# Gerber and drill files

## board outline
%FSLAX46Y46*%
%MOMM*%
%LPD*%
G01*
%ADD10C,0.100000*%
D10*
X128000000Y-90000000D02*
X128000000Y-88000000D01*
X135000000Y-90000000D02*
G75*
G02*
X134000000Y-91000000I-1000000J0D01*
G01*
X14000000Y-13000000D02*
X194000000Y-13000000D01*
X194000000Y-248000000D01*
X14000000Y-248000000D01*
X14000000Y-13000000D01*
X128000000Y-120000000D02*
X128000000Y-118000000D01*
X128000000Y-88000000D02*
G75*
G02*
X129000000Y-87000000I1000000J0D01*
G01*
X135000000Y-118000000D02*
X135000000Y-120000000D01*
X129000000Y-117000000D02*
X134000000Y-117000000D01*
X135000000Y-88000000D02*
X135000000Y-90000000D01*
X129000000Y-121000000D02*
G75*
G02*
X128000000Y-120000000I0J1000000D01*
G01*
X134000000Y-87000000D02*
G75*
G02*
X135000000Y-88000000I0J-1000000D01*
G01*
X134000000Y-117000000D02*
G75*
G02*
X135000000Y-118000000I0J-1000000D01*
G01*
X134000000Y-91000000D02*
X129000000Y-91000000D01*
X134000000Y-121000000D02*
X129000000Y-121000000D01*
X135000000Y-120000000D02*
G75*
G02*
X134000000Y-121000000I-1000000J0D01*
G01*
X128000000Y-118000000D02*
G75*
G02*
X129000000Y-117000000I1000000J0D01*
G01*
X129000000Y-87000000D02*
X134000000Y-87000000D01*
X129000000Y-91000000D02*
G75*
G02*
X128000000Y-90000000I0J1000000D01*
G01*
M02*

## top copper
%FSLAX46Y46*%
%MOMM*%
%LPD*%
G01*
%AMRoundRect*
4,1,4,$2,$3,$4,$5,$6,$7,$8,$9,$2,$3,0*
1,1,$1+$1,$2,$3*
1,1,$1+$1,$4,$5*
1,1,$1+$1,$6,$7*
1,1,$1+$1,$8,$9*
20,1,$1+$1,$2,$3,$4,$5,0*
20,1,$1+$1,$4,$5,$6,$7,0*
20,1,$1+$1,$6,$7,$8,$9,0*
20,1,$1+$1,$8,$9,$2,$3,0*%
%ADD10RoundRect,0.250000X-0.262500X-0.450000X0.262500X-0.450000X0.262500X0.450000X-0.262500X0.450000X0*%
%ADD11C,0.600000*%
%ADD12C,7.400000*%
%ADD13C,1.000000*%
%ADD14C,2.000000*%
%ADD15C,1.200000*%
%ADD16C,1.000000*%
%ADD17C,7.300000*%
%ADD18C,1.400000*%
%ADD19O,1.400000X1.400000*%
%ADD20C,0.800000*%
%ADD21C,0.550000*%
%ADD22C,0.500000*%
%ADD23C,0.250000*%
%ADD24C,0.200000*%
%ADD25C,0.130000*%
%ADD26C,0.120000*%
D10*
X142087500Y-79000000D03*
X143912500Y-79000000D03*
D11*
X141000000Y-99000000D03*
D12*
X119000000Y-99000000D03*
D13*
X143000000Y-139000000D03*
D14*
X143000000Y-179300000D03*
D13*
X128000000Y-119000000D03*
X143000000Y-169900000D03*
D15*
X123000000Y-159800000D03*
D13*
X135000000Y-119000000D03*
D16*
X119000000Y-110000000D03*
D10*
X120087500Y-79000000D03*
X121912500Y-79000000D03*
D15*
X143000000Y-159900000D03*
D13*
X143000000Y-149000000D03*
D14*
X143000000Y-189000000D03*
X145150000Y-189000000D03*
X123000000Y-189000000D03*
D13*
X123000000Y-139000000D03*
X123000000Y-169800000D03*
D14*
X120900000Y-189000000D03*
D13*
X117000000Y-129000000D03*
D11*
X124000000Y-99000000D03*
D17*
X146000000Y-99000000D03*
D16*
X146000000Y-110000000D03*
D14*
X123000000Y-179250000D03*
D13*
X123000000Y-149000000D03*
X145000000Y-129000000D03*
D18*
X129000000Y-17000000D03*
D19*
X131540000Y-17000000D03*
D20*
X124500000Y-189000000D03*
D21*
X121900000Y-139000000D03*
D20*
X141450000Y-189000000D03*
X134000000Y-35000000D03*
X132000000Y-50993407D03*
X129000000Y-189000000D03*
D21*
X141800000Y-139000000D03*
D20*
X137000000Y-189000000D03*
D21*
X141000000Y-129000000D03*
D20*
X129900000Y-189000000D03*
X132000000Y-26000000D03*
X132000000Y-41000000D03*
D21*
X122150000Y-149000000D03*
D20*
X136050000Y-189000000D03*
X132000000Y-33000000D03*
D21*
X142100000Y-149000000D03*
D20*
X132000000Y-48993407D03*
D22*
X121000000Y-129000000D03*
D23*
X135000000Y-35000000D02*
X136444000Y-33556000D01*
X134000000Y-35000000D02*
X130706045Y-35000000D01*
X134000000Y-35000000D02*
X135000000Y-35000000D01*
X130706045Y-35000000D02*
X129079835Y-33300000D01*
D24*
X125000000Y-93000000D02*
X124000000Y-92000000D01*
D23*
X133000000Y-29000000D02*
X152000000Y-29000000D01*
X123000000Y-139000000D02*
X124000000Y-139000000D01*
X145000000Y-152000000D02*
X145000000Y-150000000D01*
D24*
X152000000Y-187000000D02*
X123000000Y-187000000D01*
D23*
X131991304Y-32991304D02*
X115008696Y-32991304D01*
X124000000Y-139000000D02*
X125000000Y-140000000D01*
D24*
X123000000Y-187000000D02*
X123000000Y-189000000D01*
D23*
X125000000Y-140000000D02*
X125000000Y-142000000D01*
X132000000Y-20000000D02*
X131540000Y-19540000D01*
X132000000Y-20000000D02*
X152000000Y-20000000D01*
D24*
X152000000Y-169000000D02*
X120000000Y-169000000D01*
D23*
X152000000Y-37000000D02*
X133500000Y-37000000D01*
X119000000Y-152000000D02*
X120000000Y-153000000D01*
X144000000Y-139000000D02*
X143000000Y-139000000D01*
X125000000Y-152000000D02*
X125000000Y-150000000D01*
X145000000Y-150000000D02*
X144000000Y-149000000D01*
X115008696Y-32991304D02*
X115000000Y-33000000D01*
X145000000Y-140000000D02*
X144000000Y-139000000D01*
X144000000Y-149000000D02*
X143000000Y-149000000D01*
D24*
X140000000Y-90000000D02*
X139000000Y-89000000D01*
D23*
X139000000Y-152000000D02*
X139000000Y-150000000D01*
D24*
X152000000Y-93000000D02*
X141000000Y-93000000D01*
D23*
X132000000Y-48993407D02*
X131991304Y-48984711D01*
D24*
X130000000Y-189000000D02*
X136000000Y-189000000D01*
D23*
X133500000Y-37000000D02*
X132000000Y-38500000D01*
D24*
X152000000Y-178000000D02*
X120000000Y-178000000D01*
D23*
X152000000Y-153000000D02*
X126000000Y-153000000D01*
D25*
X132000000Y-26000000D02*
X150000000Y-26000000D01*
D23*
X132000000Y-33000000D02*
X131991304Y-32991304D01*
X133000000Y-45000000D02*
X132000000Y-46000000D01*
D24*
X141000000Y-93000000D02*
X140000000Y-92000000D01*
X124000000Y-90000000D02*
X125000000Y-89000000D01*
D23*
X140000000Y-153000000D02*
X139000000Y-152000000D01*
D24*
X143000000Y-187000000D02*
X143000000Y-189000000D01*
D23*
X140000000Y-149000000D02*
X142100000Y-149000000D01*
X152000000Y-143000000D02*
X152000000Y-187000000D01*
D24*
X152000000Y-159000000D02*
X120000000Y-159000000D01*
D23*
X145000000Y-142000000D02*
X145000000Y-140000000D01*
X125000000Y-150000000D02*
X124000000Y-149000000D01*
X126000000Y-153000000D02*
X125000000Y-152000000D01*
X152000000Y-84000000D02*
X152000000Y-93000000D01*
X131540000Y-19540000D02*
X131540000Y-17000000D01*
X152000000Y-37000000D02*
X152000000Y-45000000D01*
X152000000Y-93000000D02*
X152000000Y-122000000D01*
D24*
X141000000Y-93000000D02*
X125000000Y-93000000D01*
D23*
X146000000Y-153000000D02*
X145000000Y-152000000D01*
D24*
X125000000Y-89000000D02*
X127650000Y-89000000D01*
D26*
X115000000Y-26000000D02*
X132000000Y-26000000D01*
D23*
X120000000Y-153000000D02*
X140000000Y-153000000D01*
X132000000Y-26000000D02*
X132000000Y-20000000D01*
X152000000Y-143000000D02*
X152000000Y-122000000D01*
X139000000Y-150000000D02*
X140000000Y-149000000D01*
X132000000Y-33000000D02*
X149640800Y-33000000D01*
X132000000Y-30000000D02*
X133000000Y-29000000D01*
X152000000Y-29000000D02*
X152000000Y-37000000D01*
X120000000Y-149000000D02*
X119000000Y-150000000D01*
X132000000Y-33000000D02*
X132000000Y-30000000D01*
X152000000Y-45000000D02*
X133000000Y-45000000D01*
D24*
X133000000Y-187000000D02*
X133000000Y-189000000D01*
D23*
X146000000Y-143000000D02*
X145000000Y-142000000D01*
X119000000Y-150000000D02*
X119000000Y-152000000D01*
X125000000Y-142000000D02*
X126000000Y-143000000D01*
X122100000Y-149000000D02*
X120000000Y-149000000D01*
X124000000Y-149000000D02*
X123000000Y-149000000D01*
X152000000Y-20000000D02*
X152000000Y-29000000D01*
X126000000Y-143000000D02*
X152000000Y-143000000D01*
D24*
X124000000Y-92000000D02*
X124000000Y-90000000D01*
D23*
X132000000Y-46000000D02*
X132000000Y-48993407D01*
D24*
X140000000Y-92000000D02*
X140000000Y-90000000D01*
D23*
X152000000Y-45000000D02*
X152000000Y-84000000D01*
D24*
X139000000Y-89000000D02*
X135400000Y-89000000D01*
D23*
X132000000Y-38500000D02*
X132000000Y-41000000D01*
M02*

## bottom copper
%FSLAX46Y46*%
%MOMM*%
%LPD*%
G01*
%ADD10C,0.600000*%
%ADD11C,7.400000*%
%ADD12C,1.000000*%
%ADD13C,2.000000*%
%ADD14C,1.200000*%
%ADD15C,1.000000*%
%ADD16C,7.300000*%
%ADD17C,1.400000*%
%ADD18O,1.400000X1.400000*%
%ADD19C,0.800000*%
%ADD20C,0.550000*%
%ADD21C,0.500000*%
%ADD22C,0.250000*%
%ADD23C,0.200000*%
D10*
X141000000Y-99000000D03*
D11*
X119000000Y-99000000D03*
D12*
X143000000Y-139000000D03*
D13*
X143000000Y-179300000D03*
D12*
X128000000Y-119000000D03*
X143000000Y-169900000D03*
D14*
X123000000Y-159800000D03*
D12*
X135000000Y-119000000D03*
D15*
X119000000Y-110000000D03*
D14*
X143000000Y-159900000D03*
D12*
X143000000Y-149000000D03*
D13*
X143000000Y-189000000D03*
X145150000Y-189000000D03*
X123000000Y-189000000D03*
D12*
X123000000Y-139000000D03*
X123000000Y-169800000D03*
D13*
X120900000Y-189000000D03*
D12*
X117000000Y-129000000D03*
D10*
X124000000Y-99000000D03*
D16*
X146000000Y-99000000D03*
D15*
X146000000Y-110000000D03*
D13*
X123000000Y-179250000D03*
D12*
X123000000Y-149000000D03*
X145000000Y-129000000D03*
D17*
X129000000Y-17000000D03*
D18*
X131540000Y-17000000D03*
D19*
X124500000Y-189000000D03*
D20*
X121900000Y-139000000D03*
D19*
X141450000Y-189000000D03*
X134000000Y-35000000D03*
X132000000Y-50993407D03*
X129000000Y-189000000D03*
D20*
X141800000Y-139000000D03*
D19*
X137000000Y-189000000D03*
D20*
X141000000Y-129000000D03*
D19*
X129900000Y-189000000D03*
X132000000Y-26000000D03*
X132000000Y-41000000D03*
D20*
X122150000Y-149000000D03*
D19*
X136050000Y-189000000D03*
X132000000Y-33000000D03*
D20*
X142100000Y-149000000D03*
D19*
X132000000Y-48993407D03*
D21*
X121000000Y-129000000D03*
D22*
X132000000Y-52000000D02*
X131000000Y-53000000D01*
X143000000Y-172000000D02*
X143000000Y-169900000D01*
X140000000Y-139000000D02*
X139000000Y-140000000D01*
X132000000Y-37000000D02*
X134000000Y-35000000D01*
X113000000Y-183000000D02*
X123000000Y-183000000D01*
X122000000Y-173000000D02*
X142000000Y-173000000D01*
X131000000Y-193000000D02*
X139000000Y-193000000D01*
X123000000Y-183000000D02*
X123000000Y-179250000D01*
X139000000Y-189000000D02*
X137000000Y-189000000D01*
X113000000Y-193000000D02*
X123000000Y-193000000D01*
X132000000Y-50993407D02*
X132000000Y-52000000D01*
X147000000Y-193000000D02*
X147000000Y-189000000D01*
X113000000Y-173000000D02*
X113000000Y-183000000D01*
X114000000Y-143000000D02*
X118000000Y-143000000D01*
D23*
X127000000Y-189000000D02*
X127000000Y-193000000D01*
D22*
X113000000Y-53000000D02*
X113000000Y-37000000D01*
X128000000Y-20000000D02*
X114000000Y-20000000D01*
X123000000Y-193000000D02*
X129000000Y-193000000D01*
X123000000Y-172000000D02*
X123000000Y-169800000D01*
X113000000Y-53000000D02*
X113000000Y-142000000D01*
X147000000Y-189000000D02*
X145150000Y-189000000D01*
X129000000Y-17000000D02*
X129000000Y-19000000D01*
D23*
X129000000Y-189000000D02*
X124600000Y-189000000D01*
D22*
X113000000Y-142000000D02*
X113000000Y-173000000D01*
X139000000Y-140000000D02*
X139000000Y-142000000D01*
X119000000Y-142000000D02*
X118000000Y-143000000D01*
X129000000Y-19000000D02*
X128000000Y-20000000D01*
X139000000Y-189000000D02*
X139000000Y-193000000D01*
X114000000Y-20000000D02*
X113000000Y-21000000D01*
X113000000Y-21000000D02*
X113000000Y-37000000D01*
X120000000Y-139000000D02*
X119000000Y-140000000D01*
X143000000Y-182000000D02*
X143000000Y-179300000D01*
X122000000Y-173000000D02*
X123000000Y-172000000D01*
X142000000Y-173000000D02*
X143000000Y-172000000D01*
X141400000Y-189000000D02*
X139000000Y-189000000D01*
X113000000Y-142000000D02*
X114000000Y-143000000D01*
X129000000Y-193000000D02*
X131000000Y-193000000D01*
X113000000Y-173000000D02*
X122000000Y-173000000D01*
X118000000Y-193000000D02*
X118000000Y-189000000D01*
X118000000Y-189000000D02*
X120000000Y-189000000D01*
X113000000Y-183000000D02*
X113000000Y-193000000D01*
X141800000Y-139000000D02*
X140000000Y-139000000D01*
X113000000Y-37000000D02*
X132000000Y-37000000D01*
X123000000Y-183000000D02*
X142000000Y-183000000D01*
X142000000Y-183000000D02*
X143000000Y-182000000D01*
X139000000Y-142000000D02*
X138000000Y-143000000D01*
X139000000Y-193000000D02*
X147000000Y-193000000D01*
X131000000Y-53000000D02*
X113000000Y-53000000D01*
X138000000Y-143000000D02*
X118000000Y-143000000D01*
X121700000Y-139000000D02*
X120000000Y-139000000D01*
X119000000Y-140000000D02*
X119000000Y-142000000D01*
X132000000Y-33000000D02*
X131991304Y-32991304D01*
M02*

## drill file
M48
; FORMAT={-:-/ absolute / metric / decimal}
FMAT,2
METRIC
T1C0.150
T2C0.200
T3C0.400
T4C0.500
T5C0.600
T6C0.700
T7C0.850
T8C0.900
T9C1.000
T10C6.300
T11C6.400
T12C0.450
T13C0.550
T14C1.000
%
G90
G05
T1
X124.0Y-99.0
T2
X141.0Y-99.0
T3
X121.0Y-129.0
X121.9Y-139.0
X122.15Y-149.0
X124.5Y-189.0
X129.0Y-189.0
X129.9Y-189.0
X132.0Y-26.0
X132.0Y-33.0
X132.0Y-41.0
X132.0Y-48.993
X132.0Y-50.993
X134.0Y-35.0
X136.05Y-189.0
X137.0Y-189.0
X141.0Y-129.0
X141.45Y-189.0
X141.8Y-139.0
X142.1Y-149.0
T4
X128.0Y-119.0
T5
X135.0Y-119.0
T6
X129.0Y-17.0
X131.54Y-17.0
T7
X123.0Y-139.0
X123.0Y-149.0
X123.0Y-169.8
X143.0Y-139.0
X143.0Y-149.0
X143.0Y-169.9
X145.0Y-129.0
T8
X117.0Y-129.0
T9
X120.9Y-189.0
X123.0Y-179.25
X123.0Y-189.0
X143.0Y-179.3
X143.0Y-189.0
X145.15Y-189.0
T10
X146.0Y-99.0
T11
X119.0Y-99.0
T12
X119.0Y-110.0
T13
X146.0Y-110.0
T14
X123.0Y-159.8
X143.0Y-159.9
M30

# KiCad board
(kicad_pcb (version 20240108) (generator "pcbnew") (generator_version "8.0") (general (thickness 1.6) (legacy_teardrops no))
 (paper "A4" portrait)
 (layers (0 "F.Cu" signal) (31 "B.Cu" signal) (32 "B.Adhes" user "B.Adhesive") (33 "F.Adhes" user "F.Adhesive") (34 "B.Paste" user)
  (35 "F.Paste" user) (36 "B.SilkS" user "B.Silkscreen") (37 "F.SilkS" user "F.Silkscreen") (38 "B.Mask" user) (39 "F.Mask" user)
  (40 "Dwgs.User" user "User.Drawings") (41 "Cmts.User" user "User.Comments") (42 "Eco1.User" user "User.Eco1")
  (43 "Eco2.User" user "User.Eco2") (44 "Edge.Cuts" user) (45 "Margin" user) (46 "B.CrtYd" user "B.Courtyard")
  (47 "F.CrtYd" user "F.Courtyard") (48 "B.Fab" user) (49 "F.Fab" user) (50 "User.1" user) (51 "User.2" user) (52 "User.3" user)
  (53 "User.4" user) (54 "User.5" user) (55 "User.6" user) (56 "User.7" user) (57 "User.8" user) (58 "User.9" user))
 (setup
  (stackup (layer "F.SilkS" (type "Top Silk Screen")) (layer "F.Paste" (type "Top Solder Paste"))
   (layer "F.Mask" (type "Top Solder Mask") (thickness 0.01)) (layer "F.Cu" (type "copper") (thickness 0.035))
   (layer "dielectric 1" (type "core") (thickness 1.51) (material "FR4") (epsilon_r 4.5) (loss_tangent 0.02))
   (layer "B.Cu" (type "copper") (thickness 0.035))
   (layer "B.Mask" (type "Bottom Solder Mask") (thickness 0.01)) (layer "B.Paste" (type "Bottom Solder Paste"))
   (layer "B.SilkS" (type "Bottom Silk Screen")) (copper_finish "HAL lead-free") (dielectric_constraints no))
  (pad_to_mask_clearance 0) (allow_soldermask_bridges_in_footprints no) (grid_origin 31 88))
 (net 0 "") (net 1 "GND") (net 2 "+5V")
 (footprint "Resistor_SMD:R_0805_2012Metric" (layer "F.Cu") (at 143 79)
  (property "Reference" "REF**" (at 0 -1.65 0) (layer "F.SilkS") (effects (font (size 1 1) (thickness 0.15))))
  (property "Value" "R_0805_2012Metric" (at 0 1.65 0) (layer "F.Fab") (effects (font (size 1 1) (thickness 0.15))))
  (pad "1" smd roundrect (at -0.9125 0) (size 1.025 1.4) (layers "F.Cu" "F.Paste" "F.Mask") (roundrect_rratio 0.243902))
  (pad "2" smd roundrect (at 0.9125 0) (size 1.025 1.4) (layers "F.Cu" "F.Paste" "F.Mask") (roundrect_rratio 0.243902)))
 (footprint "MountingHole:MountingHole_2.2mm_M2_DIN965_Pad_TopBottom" (layer "F.Cu") (at 141 99)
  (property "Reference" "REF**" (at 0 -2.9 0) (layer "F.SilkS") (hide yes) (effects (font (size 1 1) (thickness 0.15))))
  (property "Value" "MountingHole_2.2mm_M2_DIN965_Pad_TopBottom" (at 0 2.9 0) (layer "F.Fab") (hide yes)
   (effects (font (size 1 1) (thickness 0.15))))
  (pad "1" thru_hole circle (at 0 0) (size 0.6 0.6) (drill 0.2) (layers "*.Cu" "*.Mask") (remove_unused_layers no)))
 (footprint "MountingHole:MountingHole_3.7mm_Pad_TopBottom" (layer "F.Cu") (at 119 99)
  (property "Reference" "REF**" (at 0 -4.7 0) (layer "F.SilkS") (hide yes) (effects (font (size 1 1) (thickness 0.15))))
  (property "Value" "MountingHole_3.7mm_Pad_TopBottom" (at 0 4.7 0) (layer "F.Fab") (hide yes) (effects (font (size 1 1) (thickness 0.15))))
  (pad "1" thru_hole circle (at 0 0) (size 7.4 7.4) (drill 6.4) (layers "*.Cu" "*.Mask") (remove_unused_layers no)))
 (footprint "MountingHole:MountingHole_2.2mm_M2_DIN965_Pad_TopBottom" (layer "F.Cu") (at 143 139)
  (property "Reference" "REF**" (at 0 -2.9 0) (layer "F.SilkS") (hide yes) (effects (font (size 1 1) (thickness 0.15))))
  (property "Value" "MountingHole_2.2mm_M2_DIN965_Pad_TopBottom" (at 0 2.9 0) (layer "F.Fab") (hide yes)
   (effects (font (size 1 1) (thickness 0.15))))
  (pad "1" thru_hole circle (at 0 0) (size 1 1) (drill 0.85) (layers "*.Cu" "*.Mask") (remove_unused_layers no) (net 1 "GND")))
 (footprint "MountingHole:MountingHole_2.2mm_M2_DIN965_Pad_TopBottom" (layer "F.Cu") (at 143 179.3)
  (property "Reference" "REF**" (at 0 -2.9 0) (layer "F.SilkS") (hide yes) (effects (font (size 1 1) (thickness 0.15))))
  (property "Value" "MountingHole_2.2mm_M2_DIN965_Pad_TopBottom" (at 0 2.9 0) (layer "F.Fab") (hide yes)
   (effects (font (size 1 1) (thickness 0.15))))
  (pad "1" thru_hole circle (at 0 0) (size 2 2) (drill 1) (layers "*.Cu" "*.Mask") (remove_unused_layers no) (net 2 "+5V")))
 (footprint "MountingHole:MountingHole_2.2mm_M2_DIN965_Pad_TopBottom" (layer "F.Cu") (at 128 119)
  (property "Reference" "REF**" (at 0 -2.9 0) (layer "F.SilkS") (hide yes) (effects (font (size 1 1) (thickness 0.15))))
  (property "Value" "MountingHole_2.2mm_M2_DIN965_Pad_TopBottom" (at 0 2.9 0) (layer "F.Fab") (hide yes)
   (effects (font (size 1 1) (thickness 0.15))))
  (pad "1" thru_hole circle (at 0 0) (size 1 1) (drill 0.5) (layers "*.Cu" "*.Mask") (remove_unused_layers no)))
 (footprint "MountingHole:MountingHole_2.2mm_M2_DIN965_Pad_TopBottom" (layer "F.Cu") (at 143 169.9)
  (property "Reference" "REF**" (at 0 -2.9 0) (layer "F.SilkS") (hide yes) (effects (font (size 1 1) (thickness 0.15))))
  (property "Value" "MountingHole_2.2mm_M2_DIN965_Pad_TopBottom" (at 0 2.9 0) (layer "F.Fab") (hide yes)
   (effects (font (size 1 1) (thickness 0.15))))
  (pad "1" thru_hole circle (at 0 0) (size 1 1) (drill 0.85) (layers "*.Cu" "*.Mask") (remove_unused_layers no) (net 2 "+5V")))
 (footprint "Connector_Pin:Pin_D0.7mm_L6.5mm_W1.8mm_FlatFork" (layer "F.Cu") (at 123 159.8)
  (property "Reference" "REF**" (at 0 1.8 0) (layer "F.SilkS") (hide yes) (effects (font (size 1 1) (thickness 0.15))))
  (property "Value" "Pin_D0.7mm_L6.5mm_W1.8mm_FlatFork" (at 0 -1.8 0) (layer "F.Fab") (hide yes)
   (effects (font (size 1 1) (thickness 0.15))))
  (pad "" np_thru_hole circle (at 0 0) (size 1.2 1.2) (drill 1) (layers "*.Cu" "*.Mask")))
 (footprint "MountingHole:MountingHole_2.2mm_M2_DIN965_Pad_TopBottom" (layer "F.Cu") (at 135 119)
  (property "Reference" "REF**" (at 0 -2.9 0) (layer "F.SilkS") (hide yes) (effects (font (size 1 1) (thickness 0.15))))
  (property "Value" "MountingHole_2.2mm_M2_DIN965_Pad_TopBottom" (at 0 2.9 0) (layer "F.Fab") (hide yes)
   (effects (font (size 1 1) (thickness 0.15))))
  (pad "1" thru_hole circle (at 0 0) (size 1 1) (drill 0.6) (layers "*.Cu" "*.Mask") (remove_unused_layers no)))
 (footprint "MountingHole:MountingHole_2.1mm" (layer "F.Cu") (at 119 110)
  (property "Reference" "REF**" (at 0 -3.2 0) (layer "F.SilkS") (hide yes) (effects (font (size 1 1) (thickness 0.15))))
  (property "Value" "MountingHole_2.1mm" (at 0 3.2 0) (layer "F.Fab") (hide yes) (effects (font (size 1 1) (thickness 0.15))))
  (pad "" np_thru_hole circle (at 0 0) (size 1 1) (drill 0.45) (layers "*.Cu" "*.Mask")))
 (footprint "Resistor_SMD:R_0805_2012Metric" (layer "F.Cu") (at 121 79)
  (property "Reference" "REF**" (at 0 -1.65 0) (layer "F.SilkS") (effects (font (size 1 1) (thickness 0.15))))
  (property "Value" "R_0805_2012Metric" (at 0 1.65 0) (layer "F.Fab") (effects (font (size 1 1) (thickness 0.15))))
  (pad "1" smd roundrect (at -0.9125 0) (size 1.025 1.4) (layers "F.Cu" "F.Paste" "F.Mask") (roundrect_rratio 0.243902))
  (pad "2" smd roundrect (at 0.9125 0) (size 1.025 1.4) (layers "F.Cu" "F.Paste" "F.Mask") (roundrect_rratio 0.243902)))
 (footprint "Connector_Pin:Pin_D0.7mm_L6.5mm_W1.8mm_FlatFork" (layer "F.Cu") (at 143 159.9)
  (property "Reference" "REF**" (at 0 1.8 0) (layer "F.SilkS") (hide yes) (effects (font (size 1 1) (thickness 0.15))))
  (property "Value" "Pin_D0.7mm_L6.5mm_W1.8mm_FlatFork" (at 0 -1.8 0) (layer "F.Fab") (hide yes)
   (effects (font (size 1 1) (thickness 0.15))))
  (pad "" np_thru_hole circle (at 0 0) (size 1.2 1.2) (drill 1) (layers "*.Cu" "*.Mask")))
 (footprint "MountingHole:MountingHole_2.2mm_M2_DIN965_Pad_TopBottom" (layer "F.Cu") (at 143 149)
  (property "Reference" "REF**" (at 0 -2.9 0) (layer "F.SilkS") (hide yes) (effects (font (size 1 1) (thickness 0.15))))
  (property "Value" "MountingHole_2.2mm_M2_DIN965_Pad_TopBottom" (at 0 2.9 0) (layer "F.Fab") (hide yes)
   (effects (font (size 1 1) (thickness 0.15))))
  (pad "1" thru_hole circle (at 0 0) (size 1 1) (drill 0.85) (layers "*.Cu" "*.Mask") (remove_unused_layers no) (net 1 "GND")))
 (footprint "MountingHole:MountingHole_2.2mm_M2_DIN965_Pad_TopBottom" (layer "F.Cu") (at 143 189)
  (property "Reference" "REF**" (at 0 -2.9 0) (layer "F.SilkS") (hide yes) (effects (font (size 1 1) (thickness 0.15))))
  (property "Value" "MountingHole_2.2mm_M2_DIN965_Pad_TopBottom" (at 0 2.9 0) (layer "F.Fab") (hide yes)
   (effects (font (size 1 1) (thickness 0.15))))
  (pad "1" thru_hole circle (at 0 0) (size 2 2) (drill 1) (layers "*.Cu" "*.Mask") (remove_unused_layers no) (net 1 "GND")))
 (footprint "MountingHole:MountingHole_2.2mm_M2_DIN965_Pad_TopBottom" (layer "F.Cu") (at 145.15 189)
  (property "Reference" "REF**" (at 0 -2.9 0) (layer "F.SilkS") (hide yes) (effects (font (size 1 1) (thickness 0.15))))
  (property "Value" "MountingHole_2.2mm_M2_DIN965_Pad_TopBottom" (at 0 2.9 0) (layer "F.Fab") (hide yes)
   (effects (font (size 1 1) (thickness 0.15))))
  (pad "1" thru_hole circle (at 0 0) (size 2 2) (drill 1) (layers "*.Cu" "*.Mask") (remove_unused_layers no) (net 2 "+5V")))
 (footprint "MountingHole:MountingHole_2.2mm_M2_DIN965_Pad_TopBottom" (layer "F.Cu") (at 123 189)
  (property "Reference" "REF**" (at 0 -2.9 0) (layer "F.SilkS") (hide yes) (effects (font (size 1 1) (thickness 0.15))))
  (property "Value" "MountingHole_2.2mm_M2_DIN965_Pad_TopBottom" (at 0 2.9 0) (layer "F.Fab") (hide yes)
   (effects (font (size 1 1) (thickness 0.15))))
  (pad "1" thru_hole circle (at 0 0) (size 2 2) (drill 1) (layers "*.Cu" "*.Mask") (remove_unused_layers no) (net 1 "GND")))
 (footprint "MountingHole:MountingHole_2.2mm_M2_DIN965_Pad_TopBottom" (layer "F.Cu") (at 123 139)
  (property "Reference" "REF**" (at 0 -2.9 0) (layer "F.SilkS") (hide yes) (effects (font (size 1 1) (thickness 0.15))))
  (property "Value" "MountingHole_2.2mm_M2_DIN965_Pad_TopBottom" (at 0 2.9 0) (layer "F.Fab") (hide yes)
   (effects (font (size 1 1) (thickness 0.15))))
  (pad "1" thru_hole circle (at 0 0) (size 1 1) (drill 0.85) (layers "*.Cu" "*.Mask") (remove_unused_layers no) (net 1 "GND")))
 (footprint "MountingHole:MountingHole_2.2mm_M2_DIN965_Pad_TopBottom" (layer "F.Cu") (at 123 169.8)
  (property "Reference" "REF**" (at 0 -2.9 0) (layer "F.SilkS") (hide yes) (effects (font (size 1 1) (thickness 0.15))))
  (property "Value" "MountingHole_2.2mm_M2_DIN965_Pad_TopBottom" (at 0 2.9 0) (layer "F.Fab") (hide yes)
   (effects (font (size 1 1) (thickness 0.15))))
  (pad "1" thru_hole circle (at 0 0) (size 1 1) (drill 0.85) (layers "*.Cu" "*.Mask") (remove_unused_layers no) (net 2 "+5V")))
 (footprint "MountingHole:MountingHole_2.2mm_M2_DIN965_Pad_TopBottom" (layer "F.Cu") (at 120.9 189)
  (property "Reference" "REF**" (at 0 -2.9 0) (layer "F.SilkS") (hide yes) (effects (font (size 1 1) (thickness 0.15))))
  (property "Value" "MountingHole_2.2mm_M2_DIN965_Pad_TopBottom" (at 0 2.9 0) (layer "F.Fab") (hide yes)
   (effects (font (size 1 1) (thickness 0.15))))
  (pad "1" thru_hole circle (at 0 0) (size 2 2) (drill 1) (layers "*.Cu" "*.Mask") (remove_unused_layers no) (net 2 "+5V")))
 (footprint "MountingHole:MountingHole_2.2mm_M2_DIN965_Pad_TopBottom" (layer "F.Cu") (at 117 129)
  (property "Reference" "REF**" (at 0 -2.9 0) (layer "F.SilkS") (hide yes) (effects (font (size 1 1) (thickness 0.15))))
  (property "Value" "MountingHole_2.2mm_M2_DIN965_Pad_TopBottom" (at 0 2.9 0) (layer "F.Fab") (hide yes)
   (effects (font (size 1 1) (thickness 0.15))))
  (pad "1" thru_hole circle (at 0 0) (size 1 1) (drill 0.9) (layers "*.Cu" "*.Mask") (remove_unused_layers no) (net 1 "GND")))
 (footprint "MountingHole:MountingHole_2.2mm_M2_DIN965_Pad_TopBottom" (layer "F.Cu") (at 124 99)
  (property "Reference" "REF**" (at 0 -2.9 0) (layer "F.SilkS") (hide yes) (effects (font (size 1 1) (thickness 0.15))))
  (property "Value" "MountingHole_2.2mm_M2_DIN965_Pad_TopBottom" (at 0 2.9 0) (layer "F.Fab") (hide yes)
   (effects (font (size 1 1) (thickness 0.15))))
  (pad "1" thru_hole circle (at 0 0) (size 0.6 0.6) (drill 0.15) (layers "*.Cu" "*.Mask") (remove_unused_layers no)))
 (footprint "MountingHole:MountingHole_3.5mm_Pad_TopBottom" (layer "F.Cu") (at 146 99)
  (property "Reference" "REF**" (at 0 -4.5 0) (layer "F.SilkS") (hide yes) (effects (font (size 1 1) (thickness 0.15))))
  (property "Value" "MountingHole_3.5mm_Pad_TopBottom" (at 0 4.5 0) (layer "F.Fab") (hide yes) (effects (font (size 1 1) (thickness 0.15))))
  (pad "1" thru_hole circle (at 0 0) (size 7.3 7.3) (drill 6.3) (layers "*.Cu" "*.Mask") (remove_unused_layers no)))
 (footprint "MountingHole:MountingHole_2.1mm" (layer "F.Cu") (at 146 110)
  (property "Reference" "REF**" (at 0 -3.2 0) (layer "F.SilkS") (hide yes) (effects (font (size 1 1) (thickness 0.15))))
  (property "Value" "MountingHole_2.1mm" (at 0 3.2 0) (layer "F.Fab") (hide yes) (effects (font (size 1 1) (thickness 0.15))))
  (pad "" np_thru_hole circle (at 0 0) (size 1 1) (drill 0.55) (layers "*.Cu" "*.Mask")))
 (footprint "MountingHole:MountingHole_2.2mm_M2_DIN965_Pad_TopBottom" (layer "F.Cu") (at 123 179.25)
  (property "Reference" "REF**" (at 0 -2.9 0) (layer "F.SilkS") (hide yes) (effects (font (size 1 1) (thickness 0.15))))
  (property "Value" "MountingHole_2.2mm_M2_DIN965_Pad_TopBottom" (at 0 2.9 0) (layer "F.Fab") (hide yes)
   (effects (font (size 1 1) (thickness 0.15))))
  (pad "1" thru_hole circle (at 0 0) (size 2 2) (drill 1) (layers "*.Cu" "*.Mask") (remove_unused_layers no) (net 2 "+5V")))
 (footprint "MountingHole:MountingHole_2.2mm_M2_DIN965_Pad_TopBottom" (layer "F.Cu") (at 123 149)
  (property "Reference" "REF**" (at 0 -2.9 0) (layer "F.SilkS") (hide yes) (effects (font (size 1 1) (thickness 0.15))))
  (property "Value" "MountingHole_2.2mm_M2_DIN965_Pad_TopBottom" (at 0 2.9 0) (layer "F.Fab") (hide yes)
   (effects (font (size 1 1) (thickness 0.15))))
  (pad "1" thru_hole circle (at 0 0) (size 1 1) (drill 0.85) (layers "*.Cu" "*.Mask") (remove_unused_layers no) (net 1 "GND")))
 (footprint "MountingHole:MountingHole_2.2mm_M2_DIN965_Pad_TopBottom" (layer "F.Cu") (at 145 129)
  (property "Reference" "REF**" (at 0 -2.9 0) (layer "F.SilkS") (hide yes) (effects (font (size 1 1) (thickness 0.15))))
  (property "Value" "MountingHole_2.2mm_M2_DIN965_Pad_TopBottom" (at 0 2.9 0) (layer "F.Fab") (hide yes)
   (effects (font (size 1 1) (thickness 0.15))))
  (pad "1" thru_hole circle (at 0 0) (size 1 1) (drill 0.85) (layers "*.Cu" "*.Mask") (remove_unused_layers no) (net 1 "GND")))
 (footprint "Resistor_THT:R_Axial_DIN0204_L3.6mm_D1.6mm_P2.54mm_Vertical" (layer "F.Cu") (at 129 17)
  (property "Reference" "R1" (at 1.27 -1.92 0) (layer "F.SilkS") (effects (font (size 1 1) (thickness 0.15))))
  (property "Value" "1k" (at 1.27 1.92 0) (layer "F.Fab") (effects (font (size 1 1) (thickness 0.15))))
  (pad "1" thru_hole circle (at 0 0) (size 1.4 1.4) (drill 0.7) (layers "*.Cu" "*.Mask") (remove_unused_layers no) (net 2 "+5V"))
  (pad "2" thru_hole oval (at 2.54 0) (size 1.4 1.4) (drill 0.7) (layers "*.Cu" "*.Mask") (remove_unused_layers no) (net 1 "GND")))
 (gr_line (start 128 90) (end 128 88) (stroke (width 0.1) (type default)) (layer "Edge.Cuts"))
 (gr_arc (start 135 90) (mid 134.707107 90.707107) (end 134 91) (stroke (width 0.1) (type default)) (layer "Edge.Cuts"))
 (gr_rect (start 14 13) (end 194 248) (locked yes) (stroke (width 0.1) (type default)) (fill none) (layer "Edge.Cuts"))
 (gr_line (start 128 120) (end 128 118) (stroke (width 0.1) (type default)) (layer "Edge.Cuts"))
 (gr_arc (start 128 88) (mid 128.292893 87.292893) (end 129 87) (stroke (width 0.1) (type default)) (layer "Edge.Cuts"))
 (gr_line (start 135 118) (end 135 120) (stroke (width 0.1) (type default)) (layer "Edge.Cuts"))
 (gr_line (start 129 117) (end 134 117) (stroke (width 0.1) (type default)) (layer "Edge.Cuts"))
 (gr_line (start 135 88) (end 135 90) (stroke (width 0.1) (type default)) (layer "Edge.Cuts"))
 (gr_arc (start 129 121) (mid 128.292893 120.707107) (end 128 120) (stroke (width 0.1) (type default)) (layer "Edge.Cuts"))
 (gr_arc (start 134 87) (mid 134.707107 87.292893) (end 135 88) (stroke (width 0.1) (type default)) (layer "Edge.Cuts"))
 (gr_arc (start 134 117) (mid 134.707107 117.292893) (end 135 118) (stroke (width 0.1) (type default)) (layer "Edge.Cuts"))
 (gr_line (start 134 91) (end 129 91) (stroke (width 0.1) (type default)) (layer "Edge.Cuts"))
 (gr_line (start 134 121) (end 129 121) (stroke (width 0.1) (type default)) (layer "Edge.Cuts"))
 (gr_arc (start 135 120) (mid 134.707107 120.707107) (end 134 121) (stroke (width 0.1) (type default)) (layer "Edge.Cuts"))
 (gr_arc (start 128 118) (mid 128.292893 117.292893) (end 129 117) (stroke (width 0.1) (type default)) (layer "Edge.Cuts"))
 (gr_line (start 129 87) (end 134 87) (stroke (width 0.1) (type default)) (layer "Edge.Cuts"))
 (gr_arc (start 129 91) (mid 128.292893 90.707107) (end 128 90) (stroke (width 0.1) (type default)) (layer "Edge.Cuts"))
 (segment (start 135 35) (end 136.444 33.556) (width 0.25) (layer "F.Cu") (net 2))
 (segment (start 134 35) (end 130.706045 35) (width 0.25) (layer "F.Cu") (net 2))
 (segment (start 134 35) (end 135 35) (width 0.25) (layer "F.Cu") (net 2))
 (segment (start 130.706045 35) (end 129.079835 33.3) (width 0.25) (layer "F.Cu") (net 2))
 (via (at 124.5 189) (size 0.8) (drill 0.4) (layers "F.Cu" "B.Cu") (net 2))
 (via (at 121.9 139) (size 0.55) (drill 0.4) (layers "F.Cu" "B.Cu") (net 2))
 (via (at 141.45 189) (size 0.8) (drill 0.4) (layers "F.Cu" "B.Cu") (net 2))
 (via (at 134 35) (size 0.8) (drill 0.4) (layers "F.Cu" "B.Cu") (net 2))
 (via (at 132 50.993407) (size 0.8) (drill 0.4) (layers "F.Cu" "B.Cu") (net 2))
 (via (at 129 189) (size 0.8) (drill 0.4) (layers "F.Cu" "B.Cu") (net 2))
 (via (at 141.8 139) (size 0.55) (drill 0.4) (layers "F.Cu" "B.Cu") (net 2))
 (via (at 137 189) (size 0.8) (drill 0.4) (layers "F.Cu" "B.Cu") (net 2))
 (segment (start 132 52) (end 131 53) (width 0.25) (layer "B.Cu") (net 2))
 (segment (start 143 172) (end 143 169.9) (width 0.25) (layer "B.Cu") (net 2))
 (segment (start 140 139) (end 139 140) (width 0.25) (layer "B.Cu") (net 2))
 (segment (start 132 37) (end 134 35) (width 0.25) (layer "B.Cu") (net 2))
 (segment (start 113 183) (end 123 183) (width 0.25) (layer "B.Cu") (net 2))
 (segment (start 122 173) (end 142 173) (width 0.25) (layer "B.Cu") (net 2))
 (segment (start 131 193) (end 139 193) (width 0.25) (layer "B.Cu") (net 2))
 (segment (start 123 183) (end 123 179.25) (width 0.25) (layer "B.Cu") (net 2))
 (segment (start 139 189) (end 137 189) (width 0.25) (layer "B.Cu") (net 2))
 (segment (start 113 193) (end 123 193) (width 0.25) (layer "B.Cu") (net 2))
 (segment (start 132 50.993407) (end 132 52) (width 0.25) (layer "B.Cu") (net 2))
 (segment (start 147 193) (end 147 189) (width 0.25) (layer "B.Cu") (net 2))
 (segment (start 113 173) (end 113 183) (width 0.25) (layer "B.Cu") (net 2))
 (segment (start 114 143) (end 118 143) (width 0.25) (layer "B.Cu") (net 2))
 (segment (start 127 189) (end 127 193) (width 0.2) (layer "B.Cu") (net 2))
 (segment (start 113 53) (end 113 37) (width 0.25) (layer "B.Cu") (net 2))
 (segment (start 128 20) (end 114 20) (width 0.25) (layer "B.Cu") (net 2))
 (segment (start 123 193) (end 129 193) (width 0.25) (layer "B.Cu") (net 2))
 (segment (start 123 172) (end 123 169.8) (width 0.25) (layer "B.Cu") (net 2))
 (segment (start 113 53) (end 113 142) (width 0.25) (layer "B.Cu") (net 2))
 (segment (start 147 189) (end 145.15 189) (width 0.25) (layer "B.Cu") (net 2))
 (segment (start 129 17) (end 129 19) (width 0.25) (layer "B.Cu") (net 2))
 (segment (start 129 189) (end 124.6 189) (width 0.2) (layer "B.Cu") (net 2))
 (segment (start 113 142) (end 113 173) (width 0.25) (layer "B.Cu") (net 2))
 (segment (start 139 140) (end 139 142) (width 0.25) (layer "B.Cu") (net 2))
 (segment (start 119 142) (end 118 143) (width 0.25) (layer "B.Cu") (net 2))
 (segment (start 129 19) (end 128 20) (width 0.25) (layer "B.Cu") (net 2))
 (segment (start 139 189) (end 139 193) (width 0.25) (layer "B.Cu") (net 2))
 (segment (start 114 20) (end 113 21) (width 0.25) (layer "B.Cu") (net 2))
 (segment (start 113 21) (end 113 37) (width 0.25) (layer "B.Cu") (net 2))
 (segment (start 120 139) (end 119 140) (width 0.25) (layer "B.Cu") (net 2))
 (segment (start 143 182) (end 143 179.3) (width 0.25) (layer "B.Cu") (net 2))
 (segment (start 122 173) (end 123 172) (width 0.25) (layer "B.Cu") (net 2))
 (segment (start 142 173) (end 143 172) (width 0.25) (layer "B.Cu") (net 2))
 (segment (start 141.4 189) (end 139 189) (width 0.25) (layer "B.Cu") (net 2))
 (segment (start 113 142) (end 114 143) (width 0.25) (layer "B.Cu") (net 2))
 (segment (start 129 193) (end 131 193) (width 0.25) (layer "B.Cu") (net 2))
 (segment (start 113 173) (end 122 173) (width 0.25) (layer "B.Cu") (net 2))
 (segment (start 118 193) (end 118 189) (width 0.25) (layer "B.Cu") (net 2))
 (segment (start 118 189) (end 120 189) (width 0.25) (layer "B.Cu") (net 2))
 (segment (start 113 183) (end 113 193) (width 0.25) (layer "B.Cu") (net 2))
 (segment (start 141.8 139) (end 140 139) (width 0.25) (layer "B.Cu") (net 2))
 (segment (start 113 37) (end 132 37) (width 0.25) (layer "B.Cu") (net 2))
 (segment (start 123 183) (end 142 183) (width 0.25) (layer "B.Cu") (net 2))
 (segment (start 142 183) (end 143 182) (width 0.25) (layer "B.Cu") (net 2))
 (segment (start 139 142) (end 138 143) (width 0.25) (layer "B.Cu") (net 2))
 (segment (start 139 193) (end 147 193) (width 0.25) (layer "B.Cu") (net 2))
 (segment (start 131 53) (end 113 53) (width 0.25) (layer "B.Cu") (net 2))
 (segment (start 138 143) (end 118 143) (width 0.25) (layer "B.Cu") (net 2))
 (segment (start 121.7 139) (end 120 139) (width 0.25) (layer "B.Cu") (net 2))
 (segment (start 119 140) (end 119 142) (width 0.25) (layer "B.Cu") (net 2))
 (segment (start 125 93) (end 124 92) (width 0.2) (layer "F.Cu") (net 1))
 (segment (start 133 29) (end 152 29) (width 0.25) (layer "F.Cu") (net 1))
 (segment (start 123 139) (end 124 139) (width 0.25) (layer "F.Cu") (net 1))
 (segment (start 145 152) (end 145 150) (width 0.25) (layer "F.Cu") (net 1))
 (segment (start 152 187) (end 123 187) (width 0.2) (layer "F.Cu") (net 1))
 (segment (start 131.991304 32.991304) (end 115.008696 32.991304) (width 0.25) (layer "F.Cu") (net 1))
 (segment (start 124 139) (end 125 140) (width 0.25) (layer "F.Cu") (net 1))
 (segment (start 123 187) (end 123 189) (width 0.2) (layer "F.Cu") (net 1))
 (segment (start 125 140) (end 125 142) (width 0.25) (layer "F.Cu") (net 1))
 (segment (start 132 20) (end 131.54 19.54) (width 0.25) (layer "F.Cu") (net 1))
 (segment (start 132 20) (end 152 20) (width 0.25) (layer "F.Cu") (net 1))
 (segment (start 152 169) (end 120 169) (width 0.2) (layer "F.Cu") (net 1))
 (segment (start 152 37) (end 133.5 37) (width 0.25) (layer "F.Cu") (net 1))
 (segment (start 119 152) (end 120 153) (width 0.25) (layer "F.Cu") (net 1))
 (segment (start 144 139) (end 143 139) (width 0.25) (layer "F.Cu") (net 1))
 (segment (start 125 152) (end 125 150) (width 0.25) (layer "F.Cu") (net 1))
 (segment (start 145 150) (end 144 149) (width 0.25) (layer "F.Cu") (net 1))
 (segment (start 115.008696 32.991304) (end 115 33) (width 0.25) (layer "F.Cu") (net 1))
 (segment (start 145 140) (end 144 139) (width 0.25) (layer "F.Cu") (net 1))
 (segment (start 144 149) (end 143 149) (width 0.25) (layer "F.Cu") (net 1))
 (segment (start 140 90) (end 139 89) (width 0.2) (layer "F.Cu") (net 1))
 (segment (start 139 152) (end 139 150) (width 0.25) (layer "F.Cu") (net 1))
 (segment (start 152 93) (end 141 93) (width 0.2) (layer "F.Cu") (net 1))
 (segment (start 132 48.993407) (end 131.991304 48.984711) (width 0.25) (layer "F.Cu") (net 1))
 (segment (start 130 189) (end 136 189) (width 0.2) (layer "F.Cu") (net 1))
 (segment (start 133.5 37) (end 132 38.5) (width 0.25) (layer "F.Cu") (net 1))
 (segment (start 152 178) (end 120 178) (width 0.2) (layer "F.Cu") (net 1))
 (segment (start 152 153) (end 126 153) (width 0.25) (layer "F.Cu") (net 1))
 (segment (start 132 26) (end 150 26) (width 0.13) (layer "F.Cu") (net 1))
 (segment (start 132 33) (end 131.991304 32.991304) (width 0.25) (layer "F.Cu") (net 1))
 (segment (start 133 45) (end 132 46) (width 0.25) (layer "F.Cu") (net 1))
 (segment (start 141 93) (end 140 92) (width 0.2) (layer "F.Cu") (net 1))
 (segment (start 124 90) (end 125 89) (width 0.2) (layer "F.Cu") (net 1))
 (segment (start 140 153) (end 139 152) (width 0.25) (layer "F.Cu") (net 1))
 (segment (start 143 187) (end 143 189) (width 0.2) (layer "F.Cu") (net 1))
 (segment (start 140 149) (end 142.1 149) (width 0.25) (layer "F.Cu") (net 1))
 (segment (start 152 143) (end 152 187) (width 0.25) (layer "F.Cu") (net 1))
 (segment (start 152 159) (end 120 159) (width 0.2) (layer "F.Cu") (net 1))
 (segment (start 145 142) (end 145 140) (width 0.25) (layer "F.Cu") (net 1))
 (segment (start 125 150) (end 124 149) (width 0.25) (layer "F.Cu") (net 1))
 (segment (start 126 153) (end 125 152) (width 0.25) (layer "F.Cu") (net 1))
 (segment (start 152 84) (end 152 93) (width 0.25) (layer "F.Cu") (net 1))
 (segment (start 131.54 19.54) (end 131.54 17) (width 0.25) (layer "F.Cu") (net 1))
 (segment (start 152 37) (end 152 45) (width 0.25) (layer "F.Cu") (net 1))
 (segment (start 152 93) (end 152 122) (width 0.25) (layer "F.Cu") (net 1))
 (segment (start 141 93) (end 125 93) (width 0.2) (layer "F.Cu") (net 1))
 (segment (start 146 153) (end 145 152) (width 0.25) (layer "F.Cu") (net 1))
 (segment (start 125 89) (end 127.65 89) (width 0.2) (layer "F.Cu") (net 1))
 (segment (start 115 26) (end 132 26) (width 0.12) (layer "F.Cu") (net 1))
 (segment (start 120 153) (end 140 153) (width 0.25) (layer "F.Cu") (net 1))
 (segment (start 132 26) (end 132 20) (width 0.25) (layer "F.Cu") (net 1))
 (segment (start 152 143) (end 152 122) (width 0.25) (layer "F.Cu") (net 1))
 (segment (start 139 150) (end 140 149) (width 0.25) (layer "F.Cu") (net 1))
 (segment (start 132 33) (end 149.6408 33) (width 0.25) (layer "F.Cu") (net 1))
 (segment (start 132 30) (end 133 29) (width 0.25) (layer "F.Cu") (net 1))
 (segment (start 152 29) (end 152 37) (width 0.25) (layer "F.Cu") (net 1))
 (segment (start 120 149) (end 119 150) (width 0.25) (layer "F.Cu") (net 1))
 (segment (start 132 33) (end 132 30) (width 0.25) (layer "F.Cu") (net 1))
 (segment (start 152 45) (end 133 45) (width 0.25) (layer "F.Cu") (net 1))
 (segment (start 133 187) (end 133 189) (width 0.2) (layer "F.Cu") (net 1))
 (segment (start 146 143) (end 145 142) (width 0.25) (layer "F.Cu") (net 1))
 (segment (start 119 150) (end 119 152) (width 0.25) (layer "F.Cu") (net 1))
 (segment (start 125 142) (end 126 143) (width 0.25) (layer "F.Cu") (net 1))
 (segment (start 122.1 149) (end 120 149) (width 0.25) (layer "F.Cu") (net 1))
 (segment (start 124 149) (end 123 149) (width 0.25) (layer "F.Cu") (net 1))
 (segment (start 152 20) (end 152 29) (width 0.25) (layer "F.Cu") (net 1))
 (segment (start 126 143) (end 152 143) (width 0.25) (layer "F.Cu") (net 1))
 (segment (start 124 92) (end 124 90) (width 0.2) (layer "F.Cu") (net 1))
 (segment (start 132 46) (end 132 48.993407) (width 0.25) (layer "F.Cu") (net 1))
 (segment (start 140 92) (end 140 90) (width 0.2) (layer "F.Cu") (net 1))
 (segment (start 152 45) (end 152 84) (width 0.25) (layer "F.Cu") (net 1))
 (segment (start 139 89) (end 135.4 89) (width 0.2) (layer "F.Cu") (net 1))
 (segment (start 132 38.5) (end 132 41) (width 0.25) (layer "F.Cu") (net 1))
 (via (at 141 129) (size 0.55) (drill 0.4) (layers "F.Cu" "B.Cu") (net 1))
 (via (at 129.9 189) (size 0.8) (drill 0.4) (layers "F.Cu" "B.Cu") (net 1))
 (via (at 132 26) (size 0.8) (drill 0.4) (layers "F.Cu" "B.Cu") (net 1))
 (via (at 132 41) (size 0.8) (drill 0.4) (layers "F.Cu" "B.Cu") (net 1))
 (via (at 122.15 149) (size 0.55) (drill 0.4) (layers "F.Cu" "B.Cu") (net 1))
 (via (at 136.05 189) (size 0.8) (drill 0.4) (layers "F.Cu" "B.Cu") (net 1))
 (via (at 132 33) (size 0.8) (drill 0.4) (layers "F.Cu" "B.Cu") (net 1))
 (via (at 142.1 149) (size 0.55) (drill 0.4) (layers "F.Cu" "B.Cu") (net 1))
 (via (at 132 48.993407) (size 0.8) (drill 0.4) (layers "F.Cu" "B.Cu") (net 1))
 (via (at 121 129) (size 0.5) (drill 0.4) (layers "F.Cu" "B.Cu") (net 1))
 (segment (start 132 33) (end 131.991304 32.991304) (width 0.25) (layer "B.Cu") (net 1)))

